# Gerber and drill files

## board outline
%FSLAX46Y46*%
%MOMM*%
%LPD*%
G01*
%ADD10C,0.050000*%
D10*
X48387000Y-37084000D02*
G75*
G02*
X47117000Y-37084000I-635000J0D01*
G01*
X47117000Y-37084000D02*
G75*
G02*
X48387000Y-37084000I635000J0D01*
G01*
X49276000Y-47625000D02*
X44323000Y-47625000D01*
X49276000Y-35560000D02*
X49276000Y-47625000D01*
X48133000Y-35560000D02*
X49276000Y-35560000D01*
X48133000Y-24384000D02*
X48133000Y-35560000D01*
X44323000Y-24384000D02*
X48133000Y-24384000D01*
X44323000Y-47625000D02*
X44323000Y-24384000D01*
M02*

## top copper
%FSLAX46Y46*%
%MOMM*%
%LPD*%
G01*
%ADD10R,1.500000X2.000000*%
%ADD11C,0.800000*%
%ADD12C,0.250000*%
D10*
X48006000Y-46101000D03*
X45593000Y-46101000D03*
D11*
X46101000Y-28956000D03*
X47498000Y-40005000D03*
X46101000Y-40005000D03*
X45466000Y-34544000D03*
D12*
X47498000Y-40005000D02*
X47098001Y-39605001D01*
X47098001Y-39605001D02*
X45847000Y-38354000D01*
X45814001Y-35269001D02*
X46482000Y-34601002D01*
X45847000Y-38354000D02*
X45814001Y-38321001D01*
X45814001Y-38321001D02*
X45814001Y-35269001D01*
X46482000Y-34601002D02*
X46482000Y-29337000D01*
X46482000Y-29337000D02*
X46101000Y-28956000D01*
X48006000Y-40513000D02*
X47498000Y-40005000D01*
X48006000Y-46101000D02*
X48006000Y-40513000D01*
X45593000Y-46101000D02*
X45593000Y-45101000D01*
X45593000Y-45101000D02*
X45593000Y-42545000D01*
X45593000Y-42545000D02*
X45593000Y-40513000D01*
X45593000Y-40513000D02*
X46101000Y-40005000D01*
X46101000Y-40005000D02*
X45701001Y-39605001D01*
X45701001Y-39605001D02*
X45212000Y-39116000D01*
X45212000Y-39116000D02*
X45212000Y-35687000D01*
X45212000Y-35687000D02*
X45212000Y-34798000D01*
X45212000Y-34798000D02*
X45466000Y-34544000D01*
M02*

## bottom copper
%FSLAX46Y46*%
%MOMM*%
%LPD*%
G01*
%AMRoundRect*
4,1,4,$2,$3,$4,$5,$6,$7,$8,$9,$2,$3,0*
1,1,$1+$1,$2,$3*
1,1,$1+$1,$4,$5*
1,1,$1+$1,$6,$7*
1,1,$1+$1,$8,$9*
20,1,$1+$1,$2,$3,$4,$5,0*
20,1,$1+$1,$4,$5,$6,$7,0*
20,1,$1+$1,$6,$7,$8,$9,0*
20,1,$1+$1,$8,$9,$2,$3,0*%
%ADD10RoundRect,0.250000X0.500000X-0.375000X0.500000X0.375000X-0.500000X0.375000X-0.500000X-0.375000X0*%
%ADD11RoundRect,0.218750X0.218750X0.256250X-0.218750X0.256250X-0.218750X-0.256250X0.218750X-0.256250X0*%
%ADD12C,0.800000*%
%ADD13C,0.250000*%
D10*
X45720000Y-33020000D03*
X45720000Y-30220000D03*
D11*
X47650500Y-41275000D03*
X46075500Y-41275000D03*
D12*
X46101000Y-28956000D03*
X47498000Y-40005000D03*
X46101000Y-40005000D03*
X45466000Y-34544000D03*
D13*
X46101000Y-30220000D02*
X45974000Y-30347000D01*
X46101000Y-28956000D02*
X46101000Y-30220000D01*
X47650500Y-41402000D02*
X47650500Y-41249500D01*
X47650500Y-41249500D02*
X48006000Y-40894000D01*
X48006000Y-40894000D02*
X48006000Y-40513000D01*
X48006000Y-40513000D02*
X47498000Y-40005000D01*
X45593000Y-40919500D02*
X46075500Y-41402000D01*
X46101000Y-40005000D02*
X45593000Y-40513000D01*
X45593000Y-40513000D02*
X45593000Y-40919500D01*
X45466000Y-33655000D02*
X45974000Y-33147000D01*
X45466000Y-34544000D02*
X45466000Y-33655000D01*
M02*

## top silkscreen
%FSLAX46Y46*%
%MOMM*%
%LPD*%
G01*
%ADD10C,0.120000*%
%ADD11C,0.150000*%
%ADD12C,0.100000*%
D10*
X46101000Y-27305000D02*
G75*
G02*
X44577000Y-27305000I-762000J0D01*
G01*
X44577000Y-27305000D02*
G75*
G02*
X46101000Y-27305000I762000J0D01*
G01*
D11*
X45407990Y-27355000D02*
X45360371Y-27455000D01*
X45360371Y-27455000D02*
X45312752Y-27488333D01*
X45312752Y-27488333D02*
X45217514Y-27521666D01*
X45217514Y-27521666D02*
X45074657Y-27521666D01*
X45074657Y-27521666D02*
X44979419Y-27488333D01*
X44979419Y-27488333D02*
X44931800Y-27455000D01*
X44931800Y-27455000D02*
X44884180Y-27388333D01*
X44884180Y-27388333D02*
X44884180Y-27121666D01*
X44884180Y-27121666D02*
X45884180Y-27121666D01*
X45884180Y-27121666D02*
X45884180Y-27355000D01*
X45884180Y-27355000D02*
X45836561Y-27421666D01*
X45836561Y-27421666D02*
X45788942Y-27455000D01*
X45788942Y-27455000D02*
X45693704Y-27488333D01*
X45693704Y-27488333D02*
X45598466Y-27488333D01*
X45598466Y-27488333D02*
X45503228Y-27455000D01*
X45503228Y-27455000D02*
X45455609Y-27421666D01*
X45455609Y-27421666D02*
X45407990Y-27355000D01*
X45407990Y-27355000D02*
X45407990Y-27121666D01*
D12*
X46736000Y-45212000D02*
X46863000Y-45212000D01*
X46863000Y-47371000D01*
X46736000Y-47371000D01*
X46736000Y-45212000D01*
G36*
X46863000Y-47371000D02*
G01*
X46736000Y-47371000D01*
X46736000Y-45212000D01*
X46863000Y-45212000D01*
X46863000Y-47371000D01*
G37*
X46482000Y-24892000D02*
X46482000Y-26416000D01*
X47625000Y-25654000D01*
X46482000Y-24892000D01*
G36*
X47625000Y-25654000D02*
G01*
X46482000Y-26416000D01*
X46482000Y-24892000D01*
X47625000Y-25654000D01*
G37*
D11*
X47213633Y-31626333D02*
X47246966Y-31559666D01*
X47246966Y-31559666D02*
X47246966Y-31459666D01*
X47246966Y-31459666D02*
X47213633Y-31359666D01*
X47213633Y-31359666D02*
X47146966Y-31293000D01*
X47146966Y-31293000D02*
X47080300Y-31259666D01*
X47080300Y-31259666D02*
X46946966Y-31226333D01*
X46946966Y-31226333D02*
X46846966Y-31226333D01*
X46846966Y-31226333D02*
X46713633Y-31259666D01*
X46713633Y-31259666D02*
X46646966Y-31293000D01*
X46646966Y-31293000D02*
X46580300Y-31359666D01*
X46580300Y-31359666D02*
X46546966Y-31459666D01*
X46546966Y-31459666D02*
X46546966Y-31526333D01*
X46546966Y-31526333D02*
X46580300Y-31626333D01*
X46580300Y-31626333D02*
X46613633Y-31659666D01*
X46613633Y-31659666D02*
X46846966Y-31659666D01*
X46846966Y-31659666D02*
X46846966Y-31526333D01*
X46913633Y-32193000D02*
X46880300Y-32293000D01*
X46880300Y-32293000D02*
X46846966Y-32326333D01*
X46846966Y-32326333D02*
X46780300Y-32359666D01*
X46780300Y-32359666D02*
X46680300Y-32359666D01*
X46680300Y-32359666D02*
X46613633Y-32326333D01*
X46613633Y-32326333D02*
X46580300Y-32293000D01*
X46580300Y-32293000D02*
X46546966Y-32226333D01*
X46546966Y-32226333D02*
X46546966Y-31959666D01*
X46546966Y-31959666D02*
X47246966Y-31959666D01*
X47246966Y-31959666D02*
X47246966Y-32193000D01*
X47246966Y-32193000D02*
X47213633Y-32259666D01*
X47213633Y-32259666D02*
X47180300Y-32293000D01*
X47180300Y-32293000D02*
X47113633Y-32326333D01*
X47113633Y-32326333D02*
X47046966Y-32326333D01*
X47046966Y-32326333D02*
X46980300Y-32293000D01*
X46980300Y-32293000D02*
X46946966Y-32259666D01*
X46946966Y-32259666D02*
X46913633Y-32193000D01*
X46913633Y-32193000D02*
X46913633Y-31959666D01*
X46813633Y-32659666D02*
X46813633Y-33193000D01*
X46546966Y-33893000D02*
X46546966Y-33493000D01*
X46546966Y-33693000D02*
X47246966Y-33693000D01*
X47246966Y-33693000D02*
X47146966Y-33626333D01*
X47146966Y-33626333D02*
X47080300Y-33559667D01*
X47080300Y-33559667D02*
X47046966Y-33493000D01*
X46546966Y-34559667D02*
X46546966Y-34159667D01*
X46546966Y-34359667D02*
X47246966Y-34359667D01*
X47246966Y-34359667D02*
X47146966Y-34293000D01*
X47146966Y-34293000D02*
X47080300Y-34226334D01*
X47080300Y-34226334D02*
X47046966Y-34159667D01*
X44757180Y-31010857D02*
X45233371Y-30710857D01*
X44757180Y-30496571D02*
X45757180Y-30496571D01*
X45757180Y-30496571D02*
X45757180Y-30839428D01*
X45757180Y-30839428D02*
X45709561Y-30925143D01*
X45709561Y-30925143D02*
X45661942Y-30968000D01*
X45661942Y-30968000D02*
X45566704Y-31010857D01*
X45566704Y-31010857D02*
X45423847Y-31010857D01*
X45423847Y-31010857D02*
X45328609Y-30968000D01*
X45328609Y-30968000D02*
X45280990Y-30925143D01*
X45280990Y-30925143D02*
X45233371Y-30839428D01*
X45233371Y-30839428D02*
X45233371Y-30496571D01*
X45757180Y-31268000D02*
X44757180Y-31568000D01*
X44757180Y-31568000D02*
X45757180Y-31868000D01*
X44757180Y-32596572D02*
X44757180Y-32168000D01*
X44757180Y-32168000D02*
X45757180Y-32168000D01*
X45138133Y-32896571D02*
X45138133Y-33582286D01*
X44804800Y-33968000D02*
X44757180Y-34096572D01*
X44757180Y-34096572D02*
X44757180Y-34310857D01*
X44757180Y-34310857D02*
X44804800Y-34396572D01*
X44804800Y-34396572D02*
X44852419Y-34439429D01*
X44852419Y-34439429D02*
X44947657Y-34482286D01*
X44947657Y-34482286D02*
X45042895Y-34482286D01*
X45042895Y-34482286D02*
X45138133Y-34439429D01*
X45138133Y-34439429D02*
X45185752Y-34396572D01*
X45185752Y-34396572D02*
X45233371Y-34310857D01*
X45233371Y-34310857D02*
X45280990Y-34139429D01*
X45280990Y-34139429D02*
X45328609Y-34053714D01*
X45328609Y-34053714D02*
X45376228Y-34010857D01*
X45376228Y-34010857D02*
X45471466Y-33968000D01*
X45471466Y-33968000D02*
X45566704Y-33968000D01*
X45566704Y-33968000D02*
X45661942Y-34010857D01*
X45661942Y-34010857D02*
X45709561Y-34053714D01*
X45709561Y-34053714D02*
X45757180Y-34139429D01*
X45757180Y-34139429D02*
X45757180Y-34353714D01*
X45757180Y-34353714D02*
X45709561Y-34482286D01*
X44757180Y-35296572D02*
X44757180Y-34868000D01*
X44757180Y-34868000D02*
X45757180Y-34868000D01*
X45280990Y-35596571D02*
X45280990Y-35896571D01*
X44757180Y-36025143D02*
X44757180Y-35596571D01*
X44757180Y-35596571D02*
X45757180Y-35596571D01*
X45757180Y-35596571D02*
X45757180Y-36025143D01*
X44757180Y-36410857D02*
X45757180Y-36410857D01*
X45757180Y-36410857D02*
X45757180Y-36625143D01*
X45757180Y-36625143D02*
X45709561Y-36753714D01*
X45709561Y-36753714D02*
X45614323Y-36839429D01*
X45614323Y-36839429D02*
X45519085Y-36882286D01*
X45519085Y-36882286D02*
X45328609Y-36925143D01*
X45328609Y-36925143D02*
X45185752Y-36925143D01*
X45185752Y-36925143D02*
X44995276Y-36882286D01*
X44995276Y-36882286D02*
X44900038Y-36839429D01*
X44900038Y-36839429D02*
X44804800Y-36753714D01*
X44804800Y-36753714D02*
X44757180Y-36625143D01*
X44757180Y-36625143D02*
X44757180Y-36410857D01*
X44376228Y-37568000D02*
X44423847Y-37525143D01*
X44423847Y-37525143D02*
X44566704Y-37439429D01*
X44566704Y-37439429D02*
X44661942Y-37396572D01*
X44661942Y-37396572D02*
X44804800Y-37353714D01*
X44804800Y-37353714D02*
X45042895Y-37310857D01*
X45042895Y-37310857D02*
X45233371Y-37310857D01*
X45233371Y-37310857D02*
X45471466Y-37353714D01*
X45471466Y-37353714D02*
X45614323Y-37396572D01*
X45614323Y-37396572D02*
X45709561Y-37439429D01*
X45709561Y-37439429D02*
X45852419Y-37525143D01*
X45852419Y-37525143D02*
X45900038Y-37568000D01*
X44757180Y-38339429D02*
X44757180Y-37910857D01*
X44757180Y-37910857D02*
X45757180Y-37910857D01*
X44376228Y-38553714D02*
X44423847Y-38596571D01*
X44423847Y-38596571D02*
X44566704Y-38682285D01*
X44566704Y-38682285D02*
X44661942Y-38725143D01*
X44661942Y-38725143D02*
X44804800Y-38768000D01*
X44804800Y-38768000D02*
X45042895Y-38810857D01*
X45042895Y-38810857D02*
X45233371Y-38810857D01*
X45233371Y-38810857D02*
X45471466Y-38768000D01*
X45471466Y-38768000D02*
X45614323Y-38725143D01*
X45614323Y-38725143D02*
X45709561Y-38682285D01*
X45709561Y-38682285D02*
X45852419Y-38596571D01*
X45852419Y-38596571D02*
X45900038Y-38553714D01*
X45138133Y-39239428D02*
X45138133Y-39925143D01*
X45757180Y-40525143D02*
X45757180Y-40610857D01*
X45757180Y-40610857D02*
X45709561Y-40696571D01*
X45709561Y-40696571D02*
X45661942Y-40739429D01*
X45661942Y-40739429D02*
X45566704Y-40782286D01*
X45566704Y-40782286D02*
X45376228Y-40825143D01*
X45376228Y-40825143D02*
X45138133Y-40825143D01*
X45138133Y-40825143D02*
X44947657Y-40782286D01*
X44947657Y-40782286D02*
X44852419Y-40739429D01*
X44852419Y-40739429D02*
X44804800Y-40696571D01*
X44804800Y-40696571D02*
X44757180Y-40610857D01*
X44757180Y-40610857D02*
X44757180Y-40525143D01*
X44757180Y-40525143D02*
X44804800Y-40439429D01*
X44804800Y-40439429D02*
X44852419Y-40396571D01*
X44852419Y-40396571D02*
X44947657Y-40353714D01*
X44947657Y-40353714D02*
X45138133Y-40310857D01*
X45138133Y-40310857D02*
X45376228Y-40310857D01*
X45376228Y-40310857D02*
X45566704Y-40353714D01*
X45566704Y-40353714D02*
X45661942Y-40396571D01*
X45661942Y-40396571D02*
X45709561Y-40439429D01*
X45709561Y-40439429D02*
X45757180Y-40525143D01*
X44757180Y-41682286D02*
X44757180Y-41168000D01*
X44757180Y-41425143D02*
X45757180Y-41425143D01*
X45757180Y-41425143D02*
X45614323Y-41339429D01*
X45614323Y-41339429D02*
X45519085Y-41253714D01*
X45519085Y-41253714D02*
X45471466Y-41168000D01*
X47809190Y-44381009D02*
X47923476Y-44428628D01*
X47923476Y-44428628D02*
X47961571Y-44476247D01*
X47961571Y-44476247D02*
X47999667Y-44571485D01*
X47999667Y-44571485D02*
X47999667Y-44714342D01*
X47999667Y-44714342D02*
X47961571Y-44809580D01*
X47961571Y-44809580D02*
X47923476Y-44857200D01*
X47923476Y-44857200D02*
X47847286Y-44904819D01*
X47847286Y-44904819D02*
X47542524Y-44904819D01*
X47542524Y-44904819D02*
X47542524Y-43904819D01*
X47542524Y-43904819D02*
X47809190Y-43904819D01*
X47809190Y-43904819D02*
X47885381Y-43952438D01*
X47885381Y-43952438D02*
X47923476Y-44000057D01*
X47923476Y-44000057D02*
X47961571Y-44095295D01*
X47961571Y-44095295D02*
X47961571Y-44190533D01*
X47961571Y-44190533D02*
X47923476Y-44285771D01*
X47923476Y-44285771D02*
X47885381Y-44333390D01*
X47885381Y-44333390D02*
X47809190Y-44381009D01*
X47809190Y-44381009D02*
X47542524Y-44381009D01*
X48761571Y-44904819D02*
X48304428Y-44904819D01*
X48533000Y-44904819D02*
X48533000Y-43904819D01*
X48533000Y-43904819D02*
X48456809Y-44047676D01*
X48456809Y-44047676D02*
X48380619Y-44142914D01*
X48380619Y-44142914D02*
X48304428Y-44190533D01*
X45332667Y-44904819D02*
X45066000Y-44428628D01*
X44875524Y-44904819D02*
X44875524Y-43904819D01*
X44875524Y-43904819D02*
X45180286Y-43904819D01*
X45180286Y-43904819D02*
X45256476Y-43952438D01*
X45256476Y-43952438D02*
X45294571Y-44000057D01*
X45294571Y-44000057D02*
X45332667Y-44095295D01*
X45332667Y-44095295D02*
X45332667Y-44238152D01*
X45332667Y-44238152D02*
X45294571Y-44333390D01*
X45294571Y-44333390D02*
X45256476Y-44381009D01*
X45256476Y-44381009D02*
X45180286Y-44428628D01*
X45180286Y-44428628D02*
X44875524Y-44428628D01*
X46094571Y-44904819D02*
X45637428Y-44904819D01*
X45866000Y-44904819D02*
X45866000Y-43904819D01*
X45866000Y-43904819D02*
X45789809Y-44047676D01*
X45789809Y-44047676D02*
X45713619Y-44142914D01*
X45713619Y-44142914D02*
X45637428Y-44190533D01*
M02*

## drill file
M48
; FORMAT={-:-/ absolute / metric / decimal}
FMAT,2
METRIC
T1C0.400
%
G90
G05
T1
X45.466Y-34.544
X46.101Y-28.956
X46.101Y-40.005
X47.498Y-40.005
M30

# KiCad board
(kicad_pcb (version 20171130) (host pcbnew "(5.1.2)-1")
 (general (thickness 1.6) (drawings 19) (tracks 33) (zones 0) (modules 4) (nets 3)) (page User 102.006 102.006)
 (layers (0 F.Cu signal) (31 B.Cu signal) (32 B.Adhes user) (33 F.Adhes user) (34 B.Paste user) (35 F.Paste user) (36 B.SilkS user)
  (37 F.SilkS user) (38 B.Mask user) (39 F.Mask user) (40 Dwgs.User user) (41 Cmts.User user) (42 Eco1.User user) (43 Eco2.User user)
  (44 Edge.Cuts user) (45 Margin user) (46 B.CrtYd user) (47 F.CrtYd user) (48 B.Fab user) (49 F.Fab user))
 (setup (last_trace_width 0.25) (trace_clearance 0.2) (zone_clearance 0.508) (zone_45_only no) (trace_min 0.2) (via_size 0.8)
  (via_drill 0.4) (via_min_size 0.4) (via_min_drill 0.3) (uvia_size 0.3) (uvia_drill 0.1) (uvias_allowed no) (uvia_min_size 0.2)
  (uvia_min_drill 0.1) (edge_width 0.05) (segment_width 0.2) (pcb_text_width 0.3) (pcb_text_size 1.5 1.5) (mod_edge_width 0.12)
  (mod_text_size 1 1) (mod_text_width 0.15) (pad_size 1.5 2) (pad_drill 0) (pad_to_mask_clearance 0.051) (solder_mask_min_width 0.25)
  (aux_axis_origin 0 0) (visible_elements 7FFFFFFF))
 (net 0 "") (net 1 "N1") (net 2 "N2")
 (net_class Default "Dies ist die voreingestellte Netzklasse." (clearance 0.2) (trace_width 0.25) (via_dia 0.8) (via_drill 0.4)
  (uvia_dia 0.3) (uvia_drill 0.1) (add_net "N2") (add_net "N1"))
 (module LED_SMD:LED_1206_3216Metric (layer B.Cu) (at 45.72 31.62 90)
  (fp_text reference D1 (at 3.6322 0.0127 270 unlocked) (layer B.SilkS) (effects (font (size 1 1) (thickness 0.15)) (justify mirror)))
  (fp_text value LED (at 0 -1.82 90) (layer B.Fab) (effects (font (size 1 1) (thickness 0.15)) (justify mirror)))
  (pad 1 smd roundrect (at -1.4 0 90) (size 1.25 1.5) (layers B.Cu B.Paste B.Mask) (roundrect_rratio 0.2) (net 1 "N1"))
  (pad 2 smd roundrect (at 1.4 0 90) (size 1.25 1.5) (layers B.Cu B.Paste B.Mask) (roundrect_rratio 0.2) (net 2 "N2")))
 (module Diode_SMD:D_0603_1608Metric (layer B.Cu) (at 46.863 41.275 180)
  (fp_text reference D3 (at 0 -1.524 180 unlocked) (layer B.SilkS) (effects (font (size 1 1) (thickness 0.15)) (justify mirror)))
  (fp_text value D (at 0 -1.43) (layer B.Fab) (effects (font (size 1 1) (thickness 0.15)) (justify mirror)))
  (pad 1 smd roundrect (at -0.7875 0 180) (size 0.875 0.95) (layers B.Cu B.Paste B.Mask) (roundrect_rratio 0.25) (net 2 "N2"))
  (pad 2 smd roundrect (at 0.7875 0 180) (size 0.875 0.95) (layers B.Cu B.Paste B.Mask) (roundrect_rratio 0.25) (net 1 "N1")))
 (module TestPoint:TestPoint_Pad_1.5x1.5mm (layer F.Cu) (at 48.006 46.101)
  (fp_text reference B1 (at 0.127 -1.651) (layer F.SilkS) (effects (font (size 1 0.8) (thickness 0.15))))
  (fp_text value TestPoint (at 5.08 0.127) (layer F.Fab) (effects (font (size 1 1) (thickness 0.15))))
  (pad 1 smd rect (at 0 0) (size 1.5 2) (layers F.Cu F.Mask) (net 2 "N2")))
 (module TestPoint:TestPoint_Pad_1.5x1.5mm (layer F.Cu) (at 45.593 46.101)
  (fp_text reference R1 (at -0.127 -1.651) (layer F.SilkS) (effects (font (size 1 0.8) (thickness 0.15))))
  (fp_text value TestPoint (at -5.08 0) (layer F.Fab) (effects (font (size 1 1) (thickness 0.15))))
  (pad 1 smd rect (at 0 0) (size 1.5 2) (layers F.Cu F.Mask) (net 1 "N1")))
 (gr_circle (center 45.339 27.305) (end 45.339 26.543) (layer F.SilkS) (width 0.12))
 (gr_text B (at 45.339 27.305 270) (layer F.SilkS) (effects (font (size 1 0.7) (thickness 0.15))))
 (gr_poly (pts (xy 46.736 45.212) (xy 46.863 45.212) (xy 46.863 47.371) (xy 46.736 47.371)) (layer F.SilkS) (width 0.1))
 (gr_circle (center 47.752 37.084) (end 47.752 36.449) (layer Edge.Cuts) (width 0.05))
 (gr_poly (pts (xy 46.482 24.892) (xy 46.482 26.416) (xy 47.625 25.654)) (layer F.SilkS) (width 0.1))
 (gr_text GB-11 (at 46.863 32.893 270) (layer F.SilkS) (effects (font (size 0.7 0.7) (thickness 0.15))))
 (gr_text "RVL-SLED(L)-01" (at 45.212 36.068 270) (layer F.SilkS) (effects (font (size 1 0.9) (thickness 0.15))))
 (gr_line (start 49.276 47.625) (end 44.323 47.625) (layer Edge.Cuts) (width 0.05))
 (gr_line (start 49.276 35.56) (end 49.276 47.625) (layer Edge.Cuts) (width 0.05))
 (gr_line (start 48.133 35.56) (end 49.276 35.56) (layer Edge.Cuts) (width 0.05))
 (gr_line (start 48.133 24.384) (end 48.133 35.56) (layer Edge.Cuts) (width 0.05))
 (gr_line (start 44.323 24.384) (end 48.133 24.384) (layer Edge.Cuts) (width 0.05))
 (gr_line (start 44.323 47.625) (end 44.323 24.384) (layer Edge.Cuts) (width 0.05))
 (segment (start 47.498 40.005) (end 47.098001 39.605001) (width 0.25) (layer F.Cu) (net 2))
 (segment (start 47.098001 39.605001) (end 45.847 38.354) (width 0.25) (layer F.Cu) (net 2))
 (segment (start 45.814001 35.269001) (end 46.482 34.601002) (width 0.25) (layer F.Cu) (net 2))
 (segment (start 45.847 38.354) (end 45.814001 38.321001) (width 0.25) (layer F.Cu) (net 2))
 (segment (start 45.814001 38.321001) (end 45.814001 35.269001) (width 0.25) (layer F.Cu) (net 2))
 (via (at 46.101 28.956) (size 0.8) (drill 0.4) (layers F.Cu B.Cu) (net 2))
 (segment (start 46.482 34.601002) (end 46.482 29.337) (width 0.25) (layer F.Cu) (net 2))
 (segment (start 46.482 29.337) (end 46.101 28.956) (width 0.25) (layer F.Cu) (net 2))
 (segment (start 46.101 30.22) (end 45.974 30.347) (width 0.25) (layer B.Cu) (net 2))
 (segment (start 46.101 28.956) (end 46.101 30.22) (width 0.25) (layer B.Cu) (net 2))
 (segment (start 48.006 40.513) (end 47.498 40.005) (width 0.25) (layer F.Cu) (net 2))
 (segment (start 48.006 46.101) (end 48.006 40.513) (width 0.25) (layer F.Cu) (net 2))
 (segment (start 47.6505 41.402) (end 47.6505 41.2495) (width 0.25) (layer B.Cu) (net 2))
 (segment (start 47.6505 41.2495) (end 48.006 40.894) (width 0.25) (layer B.Cu) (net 2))
 (via (at 47.498 40.005) (size 0.8) (drill 0.4) (layers F.Cu B.Cu) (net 2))
 (segment (start 48.006 40.894) (end 48.006 40.513) (width 0.25) (layer B.Cu) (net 2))
 (segment (start 48.006 40.513) (end 47.498 40.005) (width 0.25) (layer B.Cu) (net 2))
 (segment (start 45.593 46.101) (end 45.593 45.101) (width 0.25) (layer F.Cu) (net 1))
 (segment (start 45.593 45.101) (end 45.593 42.545) (width 0.25) (layer F.Cu) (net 1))
 (via (at 46.101 40.005) (size 0.8) (drill 0.4) (layers F.Cu B.Cu) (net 1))
 (segment (start 45.593 42.545) (end 45.593 40.513) (width 0.25) (layer F.Cu) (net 1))
 (segment (start 45.593 40.513) (end 46.101 40.005) (width 0.25) (layer F.Cu) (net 1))
 (segment (start 46.101 40.005) (end 45.701001 39.605001) (width 0.25) (layer F.Cu) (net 1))
 (segment (start 45.701001 39.605001) (end 45.212 39.116) (width 0.25) (layer F.Cu) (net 1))
 (segment (start 45.212 39.116) (end 45.212 35.687) (width 0.25) (layer F.Cu) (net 1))
 (via (at 45.466 34.544) (size 0.8) (drill 0.4) (layers F.Cu B.Cu) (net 1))
 (segment (start 45.212 35.687) (end 45.212 34.798) (width 0.25) (layer F.Cu) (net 1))
 (segment (start 45.212 34.798) (end 45.466 34.544) (width 0.25) (layer F.Cu) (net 1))
 (segment (start 45.593 40.9195) (end 46.0755 41.402) (width 0.25) (layer B.Cu) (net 1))
 (segment (start 46.101 40.005) (end 45.593 40.513) (width 0.25) (layer B.Cu) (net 1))
 (segment (start 45.593 40.513) (end 45.593 40.9195) (width 0.25) (layer B.Cu) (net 1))
 (segment (start 45.466 33.655) (end 45.974 33.147) (width 0.25) (layer B.Cu) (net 1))
 (segment (start 45.466 34.544) (end 45.466 33.655) (width 0.25) (layer B.Cu) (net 1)))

